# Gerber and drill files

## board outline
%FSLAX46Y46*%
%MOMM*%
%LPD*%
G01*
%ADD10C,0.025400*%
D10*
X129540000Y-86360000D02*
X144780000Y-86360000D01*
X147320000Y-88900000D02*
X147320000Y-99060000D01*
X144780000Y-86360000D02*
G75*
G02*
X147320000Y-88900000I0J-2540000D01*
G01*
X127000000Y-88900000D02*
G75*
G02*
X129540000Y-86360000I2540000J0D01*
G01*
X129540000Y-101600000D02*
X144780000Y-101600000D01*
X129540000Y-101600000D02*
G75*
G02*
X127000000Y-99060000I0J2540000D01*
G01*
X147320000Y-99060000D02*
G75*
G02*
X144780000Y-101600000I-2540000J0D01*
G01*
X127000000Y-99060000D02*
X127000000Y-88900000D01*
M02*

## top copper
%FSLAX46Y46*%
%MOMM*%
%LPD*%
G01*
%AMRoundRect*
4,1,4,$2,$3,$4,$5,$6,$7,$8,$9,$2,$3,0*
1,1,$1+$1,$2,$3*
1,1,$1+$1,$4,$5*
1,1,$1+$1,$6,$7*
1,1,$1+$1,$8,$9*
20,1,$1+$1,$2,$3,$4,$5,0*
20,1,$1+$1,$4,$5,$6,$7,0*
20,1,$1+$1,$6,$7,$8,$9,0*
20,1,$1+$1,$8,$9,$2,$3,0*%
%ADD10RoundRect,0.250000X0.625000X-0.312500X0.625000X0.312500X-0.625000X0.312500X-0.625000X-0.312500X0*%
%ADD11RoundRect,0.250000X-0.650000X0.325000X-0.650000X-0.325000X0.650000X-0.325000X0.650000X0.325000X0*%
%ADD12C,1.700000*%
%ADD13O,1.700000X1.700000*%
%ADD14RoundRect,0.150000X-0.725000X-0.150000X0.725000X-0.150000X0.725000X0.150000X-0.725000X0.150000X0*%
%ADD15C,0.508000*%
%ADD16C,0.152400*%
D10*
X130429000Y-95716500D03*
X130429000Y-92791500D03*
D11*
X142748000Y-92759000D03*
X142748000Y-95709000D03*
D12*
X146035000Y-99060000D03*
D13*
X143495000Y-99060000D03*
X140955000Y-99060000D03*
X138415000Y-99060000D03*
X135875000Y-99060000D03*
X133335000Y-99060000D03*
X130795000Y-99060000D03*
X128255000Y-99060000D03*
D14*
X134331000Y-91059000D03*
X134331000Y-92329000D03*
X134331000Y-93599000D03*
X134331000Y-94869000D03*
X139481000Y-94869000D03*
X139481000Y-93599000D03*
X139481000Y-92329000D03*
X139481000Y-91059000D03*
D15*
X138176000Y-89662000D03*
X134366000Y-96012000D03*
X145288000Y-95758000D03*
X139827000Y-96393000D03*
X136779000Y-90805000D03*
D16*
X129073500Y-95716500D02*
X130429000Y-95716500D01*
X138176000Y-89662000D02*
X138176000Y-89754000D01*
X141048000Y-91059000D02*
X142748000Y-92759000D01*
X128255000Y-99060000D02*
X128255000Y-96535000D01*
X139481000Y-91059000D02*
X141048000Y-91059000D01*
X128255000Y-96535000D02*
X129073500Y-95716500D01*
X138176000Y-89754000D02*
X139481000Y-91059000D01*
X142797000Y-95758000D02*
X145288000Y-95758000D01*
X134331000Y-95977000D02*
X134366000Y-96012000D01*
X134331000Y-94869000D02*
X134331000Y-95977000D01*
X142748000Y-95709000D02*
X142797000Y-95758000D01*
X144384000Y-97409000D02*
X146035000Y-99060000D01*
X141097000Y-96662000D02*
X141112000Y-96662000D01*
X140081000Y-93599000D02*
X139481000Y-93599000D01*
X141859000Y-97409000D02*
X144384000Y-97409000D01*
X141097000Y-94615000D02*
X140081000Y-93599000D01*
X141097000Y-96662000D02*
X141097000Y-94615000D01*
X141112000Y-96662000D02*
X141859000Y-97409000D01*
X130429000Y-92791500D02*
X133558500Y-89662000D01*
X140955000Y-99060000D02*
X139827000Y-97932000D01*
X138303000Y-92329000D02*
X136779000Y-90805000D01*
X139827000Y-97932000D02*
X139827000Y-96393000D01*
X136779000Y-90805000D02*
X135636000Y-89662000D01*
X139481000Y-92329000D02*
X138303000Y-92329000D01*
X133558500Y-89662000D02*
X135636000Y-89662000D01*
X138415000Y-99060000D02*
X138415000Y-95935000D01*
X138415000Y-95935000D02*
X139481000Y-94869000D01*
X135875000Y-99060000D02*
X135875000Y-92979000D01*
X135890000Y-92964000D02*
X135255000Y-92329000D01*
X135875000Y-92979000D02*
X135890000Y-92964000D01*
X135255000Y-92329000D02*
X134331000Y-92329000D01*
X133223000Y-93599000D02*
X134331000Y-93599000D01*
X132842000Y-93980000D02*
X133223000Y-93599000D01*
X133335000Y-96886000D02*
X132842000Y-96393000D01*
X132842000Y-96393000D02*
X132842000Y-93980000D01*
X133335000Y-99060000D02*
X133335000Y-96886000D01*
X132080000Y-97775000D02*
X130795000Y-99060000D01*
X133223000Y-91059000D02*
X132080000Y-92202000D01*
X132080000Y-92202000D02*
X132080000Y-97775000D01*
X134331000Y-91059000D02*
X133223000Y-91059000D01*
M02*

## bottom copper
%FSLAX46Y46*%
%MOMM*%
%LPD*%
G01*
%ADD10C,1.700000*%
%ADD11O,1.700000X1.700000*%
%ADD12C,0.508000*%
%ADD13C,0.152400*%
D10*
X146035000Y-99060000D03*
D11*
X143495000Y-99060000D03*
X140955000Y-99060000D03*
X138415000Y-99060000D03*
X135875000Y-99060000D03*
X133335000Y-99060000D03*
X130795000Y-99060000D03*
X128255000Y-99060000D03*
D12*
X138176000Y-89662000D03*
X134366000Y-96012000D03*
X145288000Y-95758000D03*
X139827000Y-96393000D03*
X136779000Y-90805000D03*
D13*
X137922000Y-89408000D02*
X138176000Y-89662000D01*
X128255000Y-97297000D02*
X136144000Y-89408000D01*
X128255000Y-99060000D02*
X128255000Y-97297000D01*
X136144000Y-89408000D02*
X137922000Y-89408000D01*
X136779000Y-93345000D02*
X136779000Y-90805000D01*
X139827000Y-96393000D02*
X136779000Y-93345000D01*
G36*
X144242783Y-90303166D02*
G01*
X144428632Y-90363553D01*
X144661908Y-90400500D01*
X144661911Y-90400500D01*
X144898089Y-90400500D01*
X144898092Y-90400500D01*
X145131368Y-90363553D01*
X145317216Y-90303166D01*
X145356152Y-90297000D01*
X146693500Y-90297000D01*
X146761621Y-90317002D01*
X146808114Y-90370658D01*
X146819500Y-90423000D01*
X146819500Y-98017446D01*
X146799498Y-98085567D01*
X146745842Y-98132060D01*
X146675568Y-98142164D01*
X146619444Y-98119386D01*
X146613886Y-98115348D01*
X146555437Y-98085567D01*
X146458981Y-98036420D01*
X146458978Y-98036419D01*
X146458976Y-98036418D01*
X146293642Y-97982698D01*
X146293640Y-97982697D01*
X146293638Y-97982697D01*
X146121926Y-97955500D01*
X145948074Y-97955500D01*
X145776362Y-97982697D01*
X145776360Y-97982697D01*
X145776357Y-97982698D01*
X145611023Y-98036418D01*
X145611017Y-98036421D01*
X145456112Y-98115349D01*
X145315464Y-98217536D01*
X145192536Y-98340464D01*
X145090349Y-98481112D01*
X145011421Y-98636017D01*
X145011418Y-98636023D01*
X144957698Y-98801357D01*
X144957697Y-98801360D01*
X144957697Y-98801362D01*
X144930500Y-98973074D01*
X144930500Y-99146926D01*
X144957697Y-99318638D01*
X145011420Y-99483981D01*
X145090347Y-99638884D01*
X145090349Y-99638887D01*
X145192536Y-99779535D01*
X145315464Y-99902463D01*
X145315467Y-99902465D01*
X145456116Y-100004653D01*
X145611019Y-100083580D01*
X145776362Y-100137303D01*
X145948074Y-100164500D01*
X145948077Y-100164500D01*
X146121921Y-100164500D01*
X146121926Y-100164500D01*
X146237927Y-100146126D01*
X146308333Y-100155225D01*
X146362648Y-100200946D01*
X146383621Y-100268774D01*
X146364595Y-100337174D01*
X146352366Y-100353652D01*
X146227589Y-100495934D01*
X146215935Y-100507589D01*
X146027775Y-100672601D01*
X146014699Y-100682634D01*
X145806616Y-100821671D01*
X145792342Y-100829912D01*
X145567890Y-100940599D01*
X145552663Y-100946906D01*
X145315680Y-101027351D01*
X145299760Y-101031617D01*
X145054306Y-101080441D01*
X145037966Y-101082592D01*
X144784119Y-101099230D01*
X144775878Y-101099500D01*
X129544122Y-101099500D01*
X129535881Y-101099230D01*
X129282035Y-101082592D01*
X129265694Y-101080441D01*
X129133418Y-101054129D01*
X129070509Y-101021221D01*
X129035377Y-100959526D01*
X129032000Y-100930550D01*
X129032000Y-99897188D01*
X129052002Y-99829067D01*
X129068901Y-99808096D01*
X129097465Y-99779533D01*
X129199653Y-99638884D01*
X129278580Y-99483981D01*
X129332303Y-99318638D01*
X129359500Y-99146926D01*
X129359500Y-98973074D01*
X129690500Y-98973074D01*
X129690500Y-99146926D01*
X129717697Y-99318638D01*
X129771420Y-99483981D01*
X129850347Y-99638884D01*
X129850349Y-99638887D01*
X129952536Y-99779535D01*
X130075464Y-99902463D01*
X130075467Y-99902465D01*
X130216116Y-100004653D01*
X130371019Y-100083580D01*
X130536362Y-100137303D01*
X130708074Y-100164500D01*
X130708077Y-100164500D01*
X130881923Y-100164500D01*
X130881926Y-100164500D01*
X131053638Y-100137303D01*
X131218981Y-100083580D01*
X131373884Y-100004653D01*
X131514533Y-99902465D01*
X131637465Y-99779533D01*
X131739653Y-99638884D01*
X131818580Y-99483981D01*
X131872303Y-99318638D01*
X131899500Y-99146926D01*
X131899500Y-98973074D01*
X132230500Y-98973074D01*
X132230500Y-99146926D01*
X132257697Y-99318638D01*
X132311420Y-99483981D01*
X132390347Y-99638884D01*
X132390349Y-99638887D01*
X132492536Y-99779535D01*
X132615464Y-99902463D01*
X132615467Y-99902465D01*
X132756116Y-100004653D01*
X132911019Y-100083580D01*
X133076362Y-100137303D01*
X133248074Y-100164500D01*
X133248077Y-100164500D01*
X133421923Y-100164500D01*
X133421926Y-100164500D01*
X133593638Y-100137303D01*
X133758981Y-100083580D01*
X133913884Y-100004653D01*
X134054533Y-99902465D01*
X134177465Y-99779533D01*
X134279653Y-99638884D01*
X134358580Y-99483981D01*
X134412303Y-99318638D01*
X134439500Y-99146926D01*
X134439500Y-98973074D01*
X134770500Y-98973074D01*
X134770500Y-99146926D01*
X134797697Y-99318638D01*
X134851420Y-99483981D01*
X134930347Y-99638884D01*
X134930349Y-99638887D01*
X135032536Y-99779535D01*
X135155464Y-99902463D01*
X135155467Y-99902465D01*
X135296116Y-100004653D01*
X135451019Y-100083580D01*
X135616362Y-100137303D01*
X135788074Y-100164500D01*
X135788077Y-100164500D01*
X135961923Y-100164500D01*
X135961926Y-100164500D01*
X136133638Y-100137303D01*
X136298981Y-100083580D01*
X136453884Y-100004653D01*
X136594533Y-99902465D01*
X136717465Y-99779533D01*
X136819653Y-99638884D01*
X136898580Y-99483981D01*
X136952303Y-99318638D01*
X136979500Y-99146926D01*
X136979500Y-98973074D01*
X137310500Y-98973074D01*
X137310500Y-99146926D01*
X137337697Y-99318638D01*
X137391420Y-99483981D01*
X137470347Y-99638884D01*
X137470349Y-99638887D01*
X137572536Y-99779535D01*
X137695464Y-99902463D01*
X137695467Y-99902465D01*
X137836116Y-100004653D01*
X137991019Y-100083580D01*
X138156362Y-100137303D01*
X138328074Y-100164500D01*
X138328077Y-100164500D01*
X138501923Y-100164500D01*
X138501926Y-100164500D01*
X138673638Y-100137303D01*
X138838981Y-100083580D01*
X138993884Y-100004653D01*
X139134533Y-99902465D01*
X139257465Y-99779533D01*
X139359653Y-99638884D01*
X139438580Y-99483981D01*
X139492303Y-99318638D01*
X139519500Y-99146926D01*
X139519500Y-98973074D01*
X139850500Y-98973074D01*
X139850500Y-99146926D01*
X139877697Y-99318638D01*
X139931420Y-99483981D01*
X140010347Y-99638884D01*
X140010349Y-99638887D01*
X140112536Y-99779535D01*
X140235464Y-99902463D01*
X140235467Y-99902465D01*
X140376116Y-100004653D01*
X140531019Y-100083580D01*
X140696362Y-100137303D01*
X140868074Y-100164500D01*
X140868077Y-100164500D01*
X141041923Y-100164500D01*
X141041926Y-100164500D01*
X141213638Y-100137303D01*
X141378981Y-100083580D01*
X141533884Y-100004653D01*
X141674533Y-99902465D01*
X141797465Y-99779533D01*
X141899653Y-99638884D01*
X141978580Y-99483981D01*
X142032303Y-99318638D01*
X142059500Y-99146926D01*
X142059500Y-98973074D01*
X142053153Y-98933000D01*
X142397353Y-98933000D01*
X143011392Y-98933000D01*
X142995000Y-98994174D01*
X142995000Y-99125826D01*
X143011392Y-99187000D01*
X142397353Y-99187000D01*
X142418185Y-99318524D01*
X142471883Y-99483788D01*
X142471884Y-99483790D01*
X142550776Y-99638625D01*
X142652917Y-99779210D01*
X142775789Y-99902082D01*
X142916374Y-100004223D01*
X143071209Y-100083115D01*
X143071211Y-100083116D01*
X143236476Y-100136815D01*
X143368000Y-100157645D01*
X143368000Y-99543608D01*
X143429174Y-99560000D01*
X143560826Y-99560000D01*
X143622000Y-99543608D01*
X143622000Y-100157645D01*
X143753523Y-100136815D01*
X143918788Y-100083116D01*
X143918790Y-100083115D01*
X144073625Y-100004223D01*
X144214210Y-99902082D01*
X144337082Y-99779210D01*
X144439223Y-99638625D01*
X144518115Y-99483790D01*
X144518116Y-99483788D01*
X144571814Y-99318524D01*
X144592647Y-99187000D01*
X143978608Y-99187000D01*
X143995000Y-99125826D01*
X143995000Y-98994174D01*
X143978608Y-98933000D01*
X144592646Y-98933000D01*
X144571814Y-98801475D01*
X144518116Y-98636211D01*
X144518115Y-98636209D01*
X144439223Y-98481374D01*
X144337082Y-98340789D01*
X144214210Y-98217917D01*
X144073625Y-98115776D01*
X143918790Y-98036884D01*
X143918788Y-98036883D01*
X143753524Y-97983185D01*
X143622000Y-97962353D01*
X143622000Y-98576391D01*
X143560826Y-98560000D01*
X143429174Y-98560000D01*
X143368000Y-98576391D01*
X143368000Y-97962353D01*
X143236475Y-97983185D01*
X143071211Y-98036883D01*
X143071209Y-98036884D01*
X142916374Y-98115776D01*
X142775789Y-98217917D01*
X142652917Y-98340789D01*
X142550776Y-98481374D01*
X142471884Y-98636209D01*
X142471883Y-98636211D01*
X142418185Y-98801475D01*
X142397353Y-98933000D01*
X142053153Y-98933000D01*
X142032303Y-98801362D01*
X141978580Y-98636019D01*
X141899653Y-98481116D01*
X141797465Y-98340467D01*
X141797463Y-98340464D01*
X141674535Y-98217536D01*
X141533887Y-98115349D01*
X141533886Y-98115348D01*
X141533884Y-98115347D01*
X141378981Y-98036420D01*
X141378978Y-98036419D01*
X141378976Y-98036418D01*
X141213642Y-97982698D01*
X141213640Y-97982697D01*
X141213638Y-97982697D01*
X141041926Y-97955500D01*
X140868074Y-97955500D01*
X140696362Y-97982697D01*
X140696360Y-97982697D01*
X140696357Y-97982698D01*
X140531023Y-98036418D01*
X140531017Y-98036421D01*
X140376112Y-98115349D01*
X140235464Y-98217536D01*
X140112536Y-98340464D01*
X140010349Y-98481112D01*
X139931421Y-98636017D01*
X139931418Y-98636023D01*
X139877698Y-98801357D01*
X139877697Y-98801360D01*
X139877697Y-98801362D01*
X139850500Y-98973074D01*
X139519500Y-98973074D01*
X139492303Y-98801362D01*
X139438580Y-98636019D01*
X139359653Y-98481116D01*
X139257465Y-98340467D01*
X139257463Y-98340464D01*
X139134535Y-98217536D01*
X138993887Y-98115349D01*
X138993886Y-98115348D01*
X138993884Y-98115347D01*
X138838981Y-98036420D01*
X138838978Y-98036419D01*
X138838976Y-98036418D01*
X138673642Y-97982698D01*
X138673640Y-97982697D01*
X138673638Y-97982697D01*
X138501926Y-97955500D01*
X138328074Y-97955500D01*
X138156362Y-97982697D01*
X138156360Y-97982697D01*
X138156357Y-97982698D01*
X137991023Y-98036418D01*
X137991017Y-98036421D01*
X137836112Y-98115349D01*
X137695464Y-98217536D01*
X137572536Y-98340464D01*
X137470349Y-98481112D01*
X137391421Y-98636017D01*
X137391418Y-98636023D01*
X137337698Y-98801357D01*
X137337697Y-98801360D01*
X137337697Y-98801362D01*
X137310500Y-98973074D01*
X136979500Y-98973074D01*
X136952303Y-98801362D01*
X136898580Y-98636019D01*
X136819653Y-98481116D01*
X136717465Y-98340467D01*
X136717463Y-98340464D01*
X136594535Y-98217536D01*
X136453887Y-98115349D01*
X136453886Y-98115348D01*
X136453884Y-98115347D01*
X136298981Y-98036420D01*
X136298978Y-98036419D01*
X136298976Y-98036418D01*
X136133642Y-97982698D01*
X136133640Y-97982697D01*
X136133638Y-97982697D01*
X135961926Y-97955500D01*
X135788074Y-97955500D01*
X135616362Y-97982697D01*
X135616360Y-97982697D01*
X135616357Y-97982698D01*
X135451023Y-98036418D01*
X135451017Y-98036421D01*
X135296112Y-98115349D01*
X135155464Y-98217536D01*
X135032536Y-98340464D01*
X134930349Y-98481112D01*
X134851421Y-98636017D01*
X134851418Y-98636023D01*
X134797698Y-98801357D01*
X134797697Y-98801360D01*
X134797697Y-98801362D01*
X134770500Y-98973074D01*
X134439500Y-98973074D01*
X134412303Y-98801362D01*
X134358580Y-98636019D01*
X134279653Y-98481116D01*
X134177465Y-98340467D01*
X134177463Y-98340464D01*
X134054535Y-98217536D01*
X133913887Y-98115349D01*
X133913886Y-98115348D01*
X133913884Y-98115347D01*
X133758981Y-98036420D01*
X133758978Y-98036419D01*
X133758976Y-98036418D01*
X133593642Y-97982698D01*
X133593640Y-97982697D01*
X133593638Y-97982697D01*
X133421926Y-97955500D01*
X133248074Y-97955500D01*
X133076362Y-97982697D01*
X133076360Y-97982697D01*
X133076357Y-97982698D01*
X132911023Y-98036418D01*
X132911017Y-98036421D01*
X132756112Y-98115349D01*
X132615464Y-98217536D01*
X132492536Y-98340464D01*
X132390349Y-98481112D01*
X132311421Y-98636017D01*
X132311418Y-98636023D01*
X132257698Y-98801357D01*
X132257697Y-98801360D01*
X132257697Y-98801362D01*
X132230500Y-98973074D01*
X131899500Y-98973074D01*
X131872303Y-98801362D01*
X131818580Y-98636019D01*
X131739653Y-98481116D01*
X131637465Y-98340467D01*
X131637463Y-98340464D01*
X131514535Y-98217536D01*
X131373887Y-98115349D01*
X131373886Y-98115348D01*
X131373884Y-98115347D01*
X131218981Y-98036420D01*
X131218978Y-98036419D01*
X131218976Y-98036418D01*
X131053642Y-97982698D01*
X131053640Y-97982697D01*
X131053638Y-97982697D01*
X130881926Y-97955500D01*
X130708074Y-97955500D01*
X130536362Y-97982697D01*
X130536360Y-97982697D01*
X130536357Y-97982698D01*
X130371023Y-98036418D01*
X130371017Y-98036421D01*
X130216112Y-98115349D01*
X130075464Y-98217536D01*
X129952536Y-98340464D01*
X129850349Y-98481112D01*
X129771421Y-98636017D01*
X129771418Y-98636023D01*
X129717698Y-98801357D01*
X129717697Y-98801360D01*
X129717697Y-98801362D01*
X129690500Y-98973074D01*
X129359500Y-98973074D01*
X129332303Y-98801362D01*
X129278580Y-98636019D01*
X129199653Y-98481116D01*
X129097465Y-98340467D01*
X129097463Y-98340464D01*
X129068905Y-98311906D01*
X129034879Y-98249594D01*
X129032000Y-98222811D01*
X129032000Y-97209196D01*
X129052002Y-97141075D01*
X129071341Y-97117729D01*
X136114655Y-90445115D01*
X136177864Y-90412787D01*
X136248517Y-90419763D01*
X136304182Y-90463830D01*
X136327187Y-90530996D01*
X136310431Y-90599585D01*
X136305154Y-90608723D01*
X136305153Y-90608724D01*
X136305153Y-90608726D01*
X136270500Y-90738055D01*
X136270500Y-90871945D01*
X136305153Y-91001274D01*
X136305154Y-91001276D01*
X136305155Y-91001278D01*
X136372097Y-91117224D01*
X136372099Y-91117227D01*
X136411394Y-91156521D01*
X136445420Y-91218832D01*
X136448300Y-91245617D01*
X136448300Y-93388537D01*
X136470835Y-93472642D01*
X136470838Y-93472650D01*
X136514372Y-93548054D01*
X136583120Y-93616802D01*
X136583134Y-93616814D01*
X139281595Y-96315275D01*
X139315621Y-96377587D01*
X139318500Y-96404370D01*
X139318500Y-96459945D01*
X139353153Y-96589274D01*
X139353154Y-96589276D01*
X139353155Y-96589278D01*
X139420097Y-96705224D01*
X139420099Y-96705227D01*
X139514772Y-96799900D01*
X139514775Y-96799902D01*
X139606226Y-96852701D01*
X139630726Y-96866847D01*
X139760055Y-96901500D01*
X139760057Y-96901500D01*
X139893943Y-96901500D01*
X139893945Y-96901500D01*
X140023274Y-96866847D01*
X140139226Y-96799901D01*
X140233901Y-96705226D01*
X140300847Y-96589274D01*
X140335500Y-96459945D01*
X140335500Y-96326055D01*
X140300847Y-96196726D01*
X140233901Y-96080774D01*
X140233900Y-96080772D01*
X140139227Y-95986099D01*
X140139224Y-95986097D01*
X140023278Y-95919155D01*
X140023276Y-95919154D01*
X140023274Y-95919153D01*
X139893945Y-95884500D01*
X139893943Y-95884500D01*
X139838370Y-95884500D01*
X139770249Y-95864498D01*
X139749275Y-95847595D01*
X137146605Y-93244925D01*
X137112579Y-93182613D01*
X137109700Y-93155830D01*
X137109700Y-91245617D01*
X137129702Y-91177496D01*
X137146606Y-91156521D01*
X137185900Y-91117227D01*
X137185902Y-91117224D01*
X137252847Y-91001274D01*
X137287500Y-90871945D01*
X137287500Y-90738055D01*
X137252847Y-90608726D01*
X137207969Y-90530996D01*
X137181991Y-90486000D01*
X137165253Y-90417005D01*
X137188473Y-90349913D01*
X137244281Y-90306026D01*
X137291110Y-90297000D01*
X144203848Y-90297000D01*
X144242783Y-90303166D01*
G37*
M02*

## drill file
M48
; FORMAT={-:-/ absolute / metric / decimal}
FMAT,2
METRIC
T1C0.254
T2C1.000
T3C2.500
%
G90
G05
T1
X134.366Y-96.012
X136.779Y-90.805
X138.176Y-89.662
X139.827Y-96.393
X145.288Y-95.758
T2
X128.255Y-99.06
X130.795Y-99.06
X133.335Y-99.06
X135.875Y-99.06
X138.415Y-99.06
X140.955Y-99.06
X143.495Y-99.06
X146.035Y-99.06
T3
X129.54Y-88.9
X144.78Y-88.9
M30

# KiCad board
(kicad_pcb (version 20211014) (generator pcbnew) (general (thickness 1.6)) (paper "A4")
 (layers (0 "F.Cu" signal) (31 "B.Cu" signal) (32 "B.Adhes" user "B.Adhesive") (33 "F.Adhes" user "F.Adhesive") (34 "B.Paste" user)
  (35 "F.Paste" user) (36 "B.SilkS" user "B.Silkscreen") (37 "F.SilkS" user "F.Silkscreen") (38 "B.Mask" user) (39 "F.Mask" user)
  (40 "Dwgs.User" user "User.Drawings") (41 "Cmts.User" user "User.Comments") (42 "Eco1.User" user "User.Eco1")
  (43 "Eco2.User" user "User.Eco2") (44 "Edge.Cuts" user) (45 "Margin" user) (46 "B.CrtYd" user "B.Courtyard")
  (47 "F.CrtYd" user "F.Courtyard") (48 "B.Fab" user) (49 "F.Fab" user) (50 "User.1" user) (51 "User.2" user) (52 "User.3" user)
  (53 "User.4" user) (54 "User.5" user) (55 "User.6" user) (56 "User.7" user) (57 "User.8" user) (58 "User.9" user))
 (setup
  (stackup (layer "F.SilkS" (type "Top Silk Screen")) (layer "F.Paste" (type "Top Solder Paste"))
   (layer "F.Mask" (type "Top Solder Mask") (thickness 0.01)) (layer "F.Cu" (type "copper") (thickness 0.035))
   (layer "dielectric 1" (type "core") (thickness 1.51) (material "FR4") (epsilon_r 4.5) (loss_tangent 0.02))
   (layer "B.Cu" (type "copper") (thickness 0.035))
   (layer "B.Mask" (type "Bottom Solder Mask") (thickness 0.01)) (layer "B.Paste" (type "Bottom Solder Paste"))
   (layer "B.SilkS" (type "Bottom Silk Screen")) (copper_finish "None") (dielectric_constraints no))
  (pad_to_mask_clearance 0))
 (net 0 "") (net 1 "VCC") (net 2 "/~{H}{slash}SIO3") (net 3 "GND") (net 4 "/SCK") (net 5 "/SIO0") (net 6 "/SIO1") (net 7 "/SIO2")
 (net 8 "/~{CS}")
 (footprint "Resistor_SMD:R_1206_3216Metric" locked (layer "F.Cu") (at 130.429 94.254 90)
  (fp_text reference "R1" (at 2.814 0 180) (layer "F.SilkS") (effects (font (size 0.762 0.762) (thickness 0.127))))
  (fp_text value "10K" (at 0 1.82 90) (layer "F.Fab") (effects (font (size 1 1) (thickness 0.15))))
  (pad "1" smd roundrect locked (at -1.4625 0 90) (size 1.125 1.75) (layers "F.Cu" "F.Paste" "F.Mask") (roundrect_rratio 0.2222222222)
   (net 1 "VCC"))
  (pad "2" smd roundrect locked (at 1.4625 0 90) (size 1.125 1.75) (layers "F.Cu" "F.Paste" "F.Mask") (roundrect_rratio 0.2222222222)
   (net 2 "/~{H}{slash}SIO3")))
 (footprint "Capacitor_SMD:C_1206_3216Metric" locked (layer "F.Cu") (at 142.748 94.234 -90)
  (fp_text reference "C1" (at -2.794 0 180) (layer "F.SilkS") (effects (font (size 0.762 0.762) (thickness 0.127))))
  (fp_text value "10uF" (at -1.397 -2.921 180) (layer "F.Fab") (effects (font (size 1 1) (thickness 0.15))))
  (pad "1" smd roundrect locked (at -1.475 0 270) (size 1.15 1.8) (layers "F.Cu" "F.Paste" "F.Mask") (roundrect_rratio 0.2173913043)
   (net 1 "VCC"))
  (pad "2" smd roundrect locked (at 1.475 0 270) (size 1.15 1.8) (layers "F.Cu" "F.Paste" "F.Mask") (roundrect_rratio 0.2173913043)
   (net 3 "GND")))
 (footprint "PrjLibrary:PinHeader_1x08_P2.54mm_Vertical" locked (layer "F.Cu") (at 146.035 99.06 -90)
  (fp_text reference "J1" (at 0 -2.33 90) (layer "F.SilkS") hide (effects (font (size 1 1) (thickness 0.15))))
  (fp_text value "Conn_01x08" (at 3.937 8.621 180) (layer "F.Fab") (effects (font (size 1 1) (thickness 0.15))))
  (pad "1" thru_hole circle locked (at 0 0 270) (size 1.7 1.7) (drill 1) (layers *.Cu *.Mask) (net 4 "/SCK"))
  (pad "2" thru_hole oval locked (at 0 2.54 270) (size 1.7 1.7) (drill 1) (layers *.Cu *.Mask) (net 3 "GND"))
  (pad "3" thru_hole oval locked (at 0 5.08 270) (size 1.7 1.7) (drill 1) (layers *.Cu *.Mask) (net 2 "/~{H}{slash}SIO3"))
  (pad "4" thru_hole oval locked (at 0 7.62 270) (size 1.7 1.7) (drill 1) (layers *.Cu *.Mask) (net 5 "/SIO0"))
  (pad "5" thru_hole oval locked (at 0 10.16 270) (size 1.7 1.7) (drill 1) (layers *.Cu *.Mask) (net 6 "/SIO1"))
  (pad "6" thru_hole oval locked (at 0 12.7 270) (size 1.7 1.7) (drill 1) (layers *.Cu *.Mask) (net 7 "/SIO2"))
  (pad "7" thru_hole oval locked (at 0 15.24 270) (size 1.7 1.7) (drill 1) (layers *.Cu *.Mask) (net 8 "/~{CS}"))
  (pad "8" thru_hole oval locked (at 0 17.78 270) (size 1.7 1.7) (drill 1) (layers *.Cu *.Mask) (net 1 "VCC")))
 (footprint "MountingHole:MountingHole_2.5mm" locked (layer "F.Cu") (at 129.54 88.9)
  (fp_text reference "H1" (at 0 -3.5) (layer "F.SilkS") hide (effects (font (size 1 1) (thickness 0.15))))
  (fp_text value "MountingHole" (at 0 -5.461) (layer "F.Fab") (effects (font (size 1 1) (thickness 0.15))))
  (pad "" np_thru_hole circle locked (at 0 0) (size 2.5 2.5) (drill 2.5) (layers *.Cu *.Mask)))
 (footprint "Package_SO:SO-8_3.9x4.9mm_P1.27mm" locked (layer "F.Cu") (at 136.906 92.964)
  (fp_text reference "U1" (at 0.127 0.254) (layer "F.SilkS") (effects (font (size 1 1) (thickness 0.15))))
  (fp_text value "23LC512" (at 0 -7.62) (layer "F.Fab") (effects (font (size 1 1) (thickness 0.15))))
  (pad "1" smd roundrect locked (at -2.575 -1.905) (size 1.75 0.6) (layers "F.Cu" "F.Paste" "F.Mask") (roundrect_rratio 0.25)
   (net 8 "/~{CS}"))
  (pad "2" smd roundrect locked (at -2.575 -0.635) (size 1.75 0.6) (layers "F.Cu" "F.Paste" "F.Mask") (roundrect_rratio 0.25)
   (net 6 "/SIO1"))
  (pad "3" smd roundrect locked (at -2.575 0.635) (size 1.75 0.6) (layers "F.Cu" "F.Paste" "F.Mask") (roundrect_rratio 0.25) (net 7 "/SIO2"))
  (pad "4" smd roundrect locked (at -2.575 1.905) (size 1.75 0.6) (layers "F.Cu" "F.Paste" "F.Mask") (roundrect_rratio 0.25) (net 3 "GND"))
  (pad "5" smd roundrect locked (at 2.575 1.905) (size 1.75 0.6) (layers "F.Cu" "F.Paste" "F.Mask") (roundrect_rratio 0.25) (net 5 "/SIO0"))
  (pad "6" smd roundrect locked (at 2.575 0.635) (size 1.75 0.6) (layers "F.Cu" "F.Paste" "F.Mask") (roundrect_rratio 0.25) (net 4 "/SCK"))
  (pad "7" smd roundrect locked (at 2.575 -0.635) (size 1.75 0.6) (layers "F.Cu" "F.Paste" "F.Mask") (roundrect_rratio 0.25)
   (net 2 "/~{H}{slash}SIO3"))
  (pad "8" smd roundrect locked (at 2.575 -1.905) (size 1.75 0.6) (layers "F.Cu" "F.Paste" "F.Mask") (roundrect_rratio 0.25) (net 1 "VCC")))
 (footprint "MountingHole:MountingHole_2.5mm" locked (layer "F.Cu") (at 144.78 88.9)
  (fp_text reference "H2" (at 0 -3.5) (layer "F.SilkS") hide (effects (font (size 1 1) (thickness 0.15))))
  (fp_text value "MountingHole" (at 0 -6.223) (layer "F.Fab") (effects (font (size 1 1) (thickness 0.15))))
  (pad "" np_thru_hole circle locked (at 0 0) (size 2.5 2.5) (drill 2.5) (layers *.Cu *.Mask)))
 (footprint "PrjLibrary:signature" (layer "B.Cu") (at 137.100818 94.115454 180)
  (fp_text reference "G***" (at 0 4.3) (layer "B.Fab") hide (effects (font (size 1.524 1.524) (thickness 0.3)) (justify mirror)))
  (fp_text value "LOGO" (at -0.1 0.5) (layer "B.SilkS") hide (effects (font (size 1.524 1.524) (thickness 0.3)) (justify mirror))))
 (gr_line locked (start 129.54 86.36) (end 144.78 86.36) (layer "Edge.Cuts") (width 0.0254))
 (gr_line locked (start 147.32 88.9) (end 147.32 99.06) (layer "Edge.Cuts") (width 0.0254))
 (gr_arc locked (start 144.78 86.36) (mid 146.576051 87.103949) (end 147.32 88.9) (layer "Edge.Cuts") (width 0.0254))
 (gr_arc locked (start 127 88.9) (mid 127.743949 87.103949) (end 129.54 86.36) (layer "Edge.Cuts") (width 0.0254))
 (gr_line locked (start 129.54 101.6) (end 144.78 101.6) (layer "Edge.Cuts") (width 0.0254))
 (gr_arc locked (start 129.54 101.6) (mid 127.743949 100.856051) (end 127 99.06) (layer "Edge.Cuts") (width 0.0254))
 (gr_arc locked (start 147.32 99.06) (mid 146.576051 100.856051) (end 144.78 101.6) (layer "Edge.Cuts") (width 0.0254))
 (gr_line locked (start 127 99.06) (end 127 88.9) (layer "Edge.Cuts") (width 0.0254))
 (segment (start 129.0735 95.7165) (end 130.429 95.7165) (width 0.1524) (layer "F.Cu") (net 1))
 (segment (start 138.176 89.662) (end 138.176 89.754) (width 0.1524) (layer "F.Cu") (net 1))
 (segment (start 141.048 91.059) (end 142.748 92.759) (width 0.1524) (layer "F.Cu") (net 1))
 (segment (start 128.255 99.06) (end 128.255 96.535) (width 0.1524) (layer "F.Cu") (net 1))
 (segment (start 139.481 91.059) (end 141.048 91.059) (width 0.1524) (layer "F.Cu") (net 1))
 (segment (start 128.255 96.535) (end 129.0735 95.7165) (width 0.1524) (layer "F.Cu") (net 1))
 (segment (start 138.176 89.754) (end 139.481 91.059) (width 0.1524) (layer "F.Cu") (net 1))
 (via (at 138.176 89.662) (size 0.508) (drill 0.254) (layers "F.Cu" "B.Cu") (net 1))
 (segment (start 137.922 89.408) (end 138.176 89.662) (width 0.1524) (layer "B.Cu") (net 1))
 (segment (start 128.255 97.297) (end 136.144 89.408) (width 0.1524) (layer "B.Cu") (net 1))
 (segment (start 128.255 99.06) (end 128.255 97.297) (width 0.1524) (layer "B.Cu") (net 1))
 (segment (start 136.144 89.408) (end 137.922 89.408) (width 0.1524) (layer "B.Cu") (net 1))
 (segment (start 142.797 95.758) (end 145.288 95.758) (width 0.1524) (layer "F.Cu") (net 3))
 (segment (start 134.331 95.977) (end 134.366 96.012) (width 0.1524) (layer "F.Cu") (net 3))
 (segment (start 134.331 94.869) (end 134.331 95.977) (width 0.1524) (layer "F.Cu") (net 3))
 (segment (start 142.748 95.709) (end 142.797 95.758) (width 0.1524) (layer "F.Cu") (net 3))
 (via (at 134.366 96.012) (size 0.508) (drill 0.254) (layers "F.Cu" "B.Cu") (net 3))
 (via (at 145.288 95.758) (size 0.508) (drill 0.254) (layers "F.Cu" "B.Cu") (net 3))
 (segment (start 144.384 97.409) (end 146.035 99.06) (width 0.1524) (layer "F.Cu") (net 4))
 (segment (start 141.097 96.662) (end 141.112 96.662) (width 0.1524) (layer "F.Cu") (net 4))
 (segment (start 140.081 93.599) (end 139.481 93.599) (width 0.1524) (layer "F.Cu") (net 4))
 (segment (start 141.859 97.409) (end 144.384 97.409) (width 0.1524) (layer "F.Cu") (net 4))
 (segment (start 141.097 94.615) (end 140.081 93.599) (width 0.1524) (layer "F.Cu") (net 4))
 (segment (start 141.097 96.662) (end 141.097 94.615) (width 0.1524) (layer "F.Cu") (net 4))
 (segment (start 141.112 96.662) (end 141.859 97.409) (width 0.1524) (layer "F.Cu") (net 4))
 (segment (start 130.429 92.7915) (end 133.5585 89.662) (width 0.1524) (layer "F.Cu") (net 2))
 (segment (start 140.955 99.06) (end 139.827 97.932) (width 0.1524) (layer "F.Cu") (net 2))
 (segment (start 138.303 92.329) (end 136.779 90.805) (width 0.1524) (layer "F.Cu") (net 2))
 (segment (start 139.827 97.932) (end 139.827 96.393) (width 0.1524) (layer "F.Cu") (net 2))
 (segment (start 136.779 90.805) (end 135.636 89.662) (width 0.1524) (layer "F.Cu") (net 2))
 (segment (start 139.481 92.329) (end 138.303 92.329) (width 0.1524) (layer "F.Cu") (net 2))
 (segment (start 133.5585 89.662) (end 135.636 89.662) (width 0.1524) (layer "F.Cu") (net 2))
 (via (at 139.827 96.393) (size 0.508) (drill 0.254) (layers "F.Cu" "B.Cu") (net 2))
 (via (at 136.779 90.805) (size 0.508) (drill 0.254) (layers "F.Cu" "B.Cu") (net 2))
 (segment (start 136.779 93.345) (end 136.779 90.805) (width 0.1524) (layer "B.Cu") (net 2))
 (segment (start 139.827 96.393) (end 136.779 93.345) (width 0.1524) (layer "B.Cu") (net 2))
 (segment (start 138.415 99.06) (end 138.415 95.935) (width 0.1524) (layer "F.Cu") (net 5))
 (segment (start 138.415 95.935) (end 139.481 94.869) (width 0.1524) (layer "F.Cu") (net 5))
 (segment (start 135.875 99.06) (end 135.875 92.979) (width 0.1524) (layer "F.Cu") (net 6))
 (segment (start 135.89 92.964) (end 135.255 92.329) (width 0.1524) (layer "F.Cu") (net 6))
 (segment (start 135.875 92.979) (end 135.89 92.964) (width 0.1524) (layer "F.Cu") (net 6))
 (segment (start 135.255 92.329) (end 134.331 92.329) (width 0.1524) (layer "F.Cu") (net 6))
 (segment (start 133.223 93.599) (end 134.331 93.599) (width 0.1524) (layer "F.Cu") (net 7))
 (segment (start 132.842 93.98) (end 133.223 93.599) (width 0.1524) (layer "F.Cu") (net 7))
 (segment (start 133.335 96.886) (end 132.842 96.393) (width 0.1524) (layer "F.Cu") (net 7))
 (segment (start 132.842 96.393) (end 132.842 93.98) (width 0.1524) (layer "F.Cu") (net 7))
 (segment (start 133.335 99.06) (end 133.335 96.886) (width 0.1524) (layer "F.Cu") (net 7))
 (segment (start 132.08 97.775) (end 130.795 99.06) (width 0.1524) (layer "F.Cu") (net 8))
 (segment (start 133.223 91.059) (end 132.08 92.202) (width 0.1524) (layer "F.Cu") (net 8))
 (segment (start 132.08 92.202) (end 132.08 97.775) (width 0.1524) (layer "F.Cu") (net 8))
 (segment (start 134.331 91.059) (end 133.223 91.059) (width 0.1524) (layer "F.Cu") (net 8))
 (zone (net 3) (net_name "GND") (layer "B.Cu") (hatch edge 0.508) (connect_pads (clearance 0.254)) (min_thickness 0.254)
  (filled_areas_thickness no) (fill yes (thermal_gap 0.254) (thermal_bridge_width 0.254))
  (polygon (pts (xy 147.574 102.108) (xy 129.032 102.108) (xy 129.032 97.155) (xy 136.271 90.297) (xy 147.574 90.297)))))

